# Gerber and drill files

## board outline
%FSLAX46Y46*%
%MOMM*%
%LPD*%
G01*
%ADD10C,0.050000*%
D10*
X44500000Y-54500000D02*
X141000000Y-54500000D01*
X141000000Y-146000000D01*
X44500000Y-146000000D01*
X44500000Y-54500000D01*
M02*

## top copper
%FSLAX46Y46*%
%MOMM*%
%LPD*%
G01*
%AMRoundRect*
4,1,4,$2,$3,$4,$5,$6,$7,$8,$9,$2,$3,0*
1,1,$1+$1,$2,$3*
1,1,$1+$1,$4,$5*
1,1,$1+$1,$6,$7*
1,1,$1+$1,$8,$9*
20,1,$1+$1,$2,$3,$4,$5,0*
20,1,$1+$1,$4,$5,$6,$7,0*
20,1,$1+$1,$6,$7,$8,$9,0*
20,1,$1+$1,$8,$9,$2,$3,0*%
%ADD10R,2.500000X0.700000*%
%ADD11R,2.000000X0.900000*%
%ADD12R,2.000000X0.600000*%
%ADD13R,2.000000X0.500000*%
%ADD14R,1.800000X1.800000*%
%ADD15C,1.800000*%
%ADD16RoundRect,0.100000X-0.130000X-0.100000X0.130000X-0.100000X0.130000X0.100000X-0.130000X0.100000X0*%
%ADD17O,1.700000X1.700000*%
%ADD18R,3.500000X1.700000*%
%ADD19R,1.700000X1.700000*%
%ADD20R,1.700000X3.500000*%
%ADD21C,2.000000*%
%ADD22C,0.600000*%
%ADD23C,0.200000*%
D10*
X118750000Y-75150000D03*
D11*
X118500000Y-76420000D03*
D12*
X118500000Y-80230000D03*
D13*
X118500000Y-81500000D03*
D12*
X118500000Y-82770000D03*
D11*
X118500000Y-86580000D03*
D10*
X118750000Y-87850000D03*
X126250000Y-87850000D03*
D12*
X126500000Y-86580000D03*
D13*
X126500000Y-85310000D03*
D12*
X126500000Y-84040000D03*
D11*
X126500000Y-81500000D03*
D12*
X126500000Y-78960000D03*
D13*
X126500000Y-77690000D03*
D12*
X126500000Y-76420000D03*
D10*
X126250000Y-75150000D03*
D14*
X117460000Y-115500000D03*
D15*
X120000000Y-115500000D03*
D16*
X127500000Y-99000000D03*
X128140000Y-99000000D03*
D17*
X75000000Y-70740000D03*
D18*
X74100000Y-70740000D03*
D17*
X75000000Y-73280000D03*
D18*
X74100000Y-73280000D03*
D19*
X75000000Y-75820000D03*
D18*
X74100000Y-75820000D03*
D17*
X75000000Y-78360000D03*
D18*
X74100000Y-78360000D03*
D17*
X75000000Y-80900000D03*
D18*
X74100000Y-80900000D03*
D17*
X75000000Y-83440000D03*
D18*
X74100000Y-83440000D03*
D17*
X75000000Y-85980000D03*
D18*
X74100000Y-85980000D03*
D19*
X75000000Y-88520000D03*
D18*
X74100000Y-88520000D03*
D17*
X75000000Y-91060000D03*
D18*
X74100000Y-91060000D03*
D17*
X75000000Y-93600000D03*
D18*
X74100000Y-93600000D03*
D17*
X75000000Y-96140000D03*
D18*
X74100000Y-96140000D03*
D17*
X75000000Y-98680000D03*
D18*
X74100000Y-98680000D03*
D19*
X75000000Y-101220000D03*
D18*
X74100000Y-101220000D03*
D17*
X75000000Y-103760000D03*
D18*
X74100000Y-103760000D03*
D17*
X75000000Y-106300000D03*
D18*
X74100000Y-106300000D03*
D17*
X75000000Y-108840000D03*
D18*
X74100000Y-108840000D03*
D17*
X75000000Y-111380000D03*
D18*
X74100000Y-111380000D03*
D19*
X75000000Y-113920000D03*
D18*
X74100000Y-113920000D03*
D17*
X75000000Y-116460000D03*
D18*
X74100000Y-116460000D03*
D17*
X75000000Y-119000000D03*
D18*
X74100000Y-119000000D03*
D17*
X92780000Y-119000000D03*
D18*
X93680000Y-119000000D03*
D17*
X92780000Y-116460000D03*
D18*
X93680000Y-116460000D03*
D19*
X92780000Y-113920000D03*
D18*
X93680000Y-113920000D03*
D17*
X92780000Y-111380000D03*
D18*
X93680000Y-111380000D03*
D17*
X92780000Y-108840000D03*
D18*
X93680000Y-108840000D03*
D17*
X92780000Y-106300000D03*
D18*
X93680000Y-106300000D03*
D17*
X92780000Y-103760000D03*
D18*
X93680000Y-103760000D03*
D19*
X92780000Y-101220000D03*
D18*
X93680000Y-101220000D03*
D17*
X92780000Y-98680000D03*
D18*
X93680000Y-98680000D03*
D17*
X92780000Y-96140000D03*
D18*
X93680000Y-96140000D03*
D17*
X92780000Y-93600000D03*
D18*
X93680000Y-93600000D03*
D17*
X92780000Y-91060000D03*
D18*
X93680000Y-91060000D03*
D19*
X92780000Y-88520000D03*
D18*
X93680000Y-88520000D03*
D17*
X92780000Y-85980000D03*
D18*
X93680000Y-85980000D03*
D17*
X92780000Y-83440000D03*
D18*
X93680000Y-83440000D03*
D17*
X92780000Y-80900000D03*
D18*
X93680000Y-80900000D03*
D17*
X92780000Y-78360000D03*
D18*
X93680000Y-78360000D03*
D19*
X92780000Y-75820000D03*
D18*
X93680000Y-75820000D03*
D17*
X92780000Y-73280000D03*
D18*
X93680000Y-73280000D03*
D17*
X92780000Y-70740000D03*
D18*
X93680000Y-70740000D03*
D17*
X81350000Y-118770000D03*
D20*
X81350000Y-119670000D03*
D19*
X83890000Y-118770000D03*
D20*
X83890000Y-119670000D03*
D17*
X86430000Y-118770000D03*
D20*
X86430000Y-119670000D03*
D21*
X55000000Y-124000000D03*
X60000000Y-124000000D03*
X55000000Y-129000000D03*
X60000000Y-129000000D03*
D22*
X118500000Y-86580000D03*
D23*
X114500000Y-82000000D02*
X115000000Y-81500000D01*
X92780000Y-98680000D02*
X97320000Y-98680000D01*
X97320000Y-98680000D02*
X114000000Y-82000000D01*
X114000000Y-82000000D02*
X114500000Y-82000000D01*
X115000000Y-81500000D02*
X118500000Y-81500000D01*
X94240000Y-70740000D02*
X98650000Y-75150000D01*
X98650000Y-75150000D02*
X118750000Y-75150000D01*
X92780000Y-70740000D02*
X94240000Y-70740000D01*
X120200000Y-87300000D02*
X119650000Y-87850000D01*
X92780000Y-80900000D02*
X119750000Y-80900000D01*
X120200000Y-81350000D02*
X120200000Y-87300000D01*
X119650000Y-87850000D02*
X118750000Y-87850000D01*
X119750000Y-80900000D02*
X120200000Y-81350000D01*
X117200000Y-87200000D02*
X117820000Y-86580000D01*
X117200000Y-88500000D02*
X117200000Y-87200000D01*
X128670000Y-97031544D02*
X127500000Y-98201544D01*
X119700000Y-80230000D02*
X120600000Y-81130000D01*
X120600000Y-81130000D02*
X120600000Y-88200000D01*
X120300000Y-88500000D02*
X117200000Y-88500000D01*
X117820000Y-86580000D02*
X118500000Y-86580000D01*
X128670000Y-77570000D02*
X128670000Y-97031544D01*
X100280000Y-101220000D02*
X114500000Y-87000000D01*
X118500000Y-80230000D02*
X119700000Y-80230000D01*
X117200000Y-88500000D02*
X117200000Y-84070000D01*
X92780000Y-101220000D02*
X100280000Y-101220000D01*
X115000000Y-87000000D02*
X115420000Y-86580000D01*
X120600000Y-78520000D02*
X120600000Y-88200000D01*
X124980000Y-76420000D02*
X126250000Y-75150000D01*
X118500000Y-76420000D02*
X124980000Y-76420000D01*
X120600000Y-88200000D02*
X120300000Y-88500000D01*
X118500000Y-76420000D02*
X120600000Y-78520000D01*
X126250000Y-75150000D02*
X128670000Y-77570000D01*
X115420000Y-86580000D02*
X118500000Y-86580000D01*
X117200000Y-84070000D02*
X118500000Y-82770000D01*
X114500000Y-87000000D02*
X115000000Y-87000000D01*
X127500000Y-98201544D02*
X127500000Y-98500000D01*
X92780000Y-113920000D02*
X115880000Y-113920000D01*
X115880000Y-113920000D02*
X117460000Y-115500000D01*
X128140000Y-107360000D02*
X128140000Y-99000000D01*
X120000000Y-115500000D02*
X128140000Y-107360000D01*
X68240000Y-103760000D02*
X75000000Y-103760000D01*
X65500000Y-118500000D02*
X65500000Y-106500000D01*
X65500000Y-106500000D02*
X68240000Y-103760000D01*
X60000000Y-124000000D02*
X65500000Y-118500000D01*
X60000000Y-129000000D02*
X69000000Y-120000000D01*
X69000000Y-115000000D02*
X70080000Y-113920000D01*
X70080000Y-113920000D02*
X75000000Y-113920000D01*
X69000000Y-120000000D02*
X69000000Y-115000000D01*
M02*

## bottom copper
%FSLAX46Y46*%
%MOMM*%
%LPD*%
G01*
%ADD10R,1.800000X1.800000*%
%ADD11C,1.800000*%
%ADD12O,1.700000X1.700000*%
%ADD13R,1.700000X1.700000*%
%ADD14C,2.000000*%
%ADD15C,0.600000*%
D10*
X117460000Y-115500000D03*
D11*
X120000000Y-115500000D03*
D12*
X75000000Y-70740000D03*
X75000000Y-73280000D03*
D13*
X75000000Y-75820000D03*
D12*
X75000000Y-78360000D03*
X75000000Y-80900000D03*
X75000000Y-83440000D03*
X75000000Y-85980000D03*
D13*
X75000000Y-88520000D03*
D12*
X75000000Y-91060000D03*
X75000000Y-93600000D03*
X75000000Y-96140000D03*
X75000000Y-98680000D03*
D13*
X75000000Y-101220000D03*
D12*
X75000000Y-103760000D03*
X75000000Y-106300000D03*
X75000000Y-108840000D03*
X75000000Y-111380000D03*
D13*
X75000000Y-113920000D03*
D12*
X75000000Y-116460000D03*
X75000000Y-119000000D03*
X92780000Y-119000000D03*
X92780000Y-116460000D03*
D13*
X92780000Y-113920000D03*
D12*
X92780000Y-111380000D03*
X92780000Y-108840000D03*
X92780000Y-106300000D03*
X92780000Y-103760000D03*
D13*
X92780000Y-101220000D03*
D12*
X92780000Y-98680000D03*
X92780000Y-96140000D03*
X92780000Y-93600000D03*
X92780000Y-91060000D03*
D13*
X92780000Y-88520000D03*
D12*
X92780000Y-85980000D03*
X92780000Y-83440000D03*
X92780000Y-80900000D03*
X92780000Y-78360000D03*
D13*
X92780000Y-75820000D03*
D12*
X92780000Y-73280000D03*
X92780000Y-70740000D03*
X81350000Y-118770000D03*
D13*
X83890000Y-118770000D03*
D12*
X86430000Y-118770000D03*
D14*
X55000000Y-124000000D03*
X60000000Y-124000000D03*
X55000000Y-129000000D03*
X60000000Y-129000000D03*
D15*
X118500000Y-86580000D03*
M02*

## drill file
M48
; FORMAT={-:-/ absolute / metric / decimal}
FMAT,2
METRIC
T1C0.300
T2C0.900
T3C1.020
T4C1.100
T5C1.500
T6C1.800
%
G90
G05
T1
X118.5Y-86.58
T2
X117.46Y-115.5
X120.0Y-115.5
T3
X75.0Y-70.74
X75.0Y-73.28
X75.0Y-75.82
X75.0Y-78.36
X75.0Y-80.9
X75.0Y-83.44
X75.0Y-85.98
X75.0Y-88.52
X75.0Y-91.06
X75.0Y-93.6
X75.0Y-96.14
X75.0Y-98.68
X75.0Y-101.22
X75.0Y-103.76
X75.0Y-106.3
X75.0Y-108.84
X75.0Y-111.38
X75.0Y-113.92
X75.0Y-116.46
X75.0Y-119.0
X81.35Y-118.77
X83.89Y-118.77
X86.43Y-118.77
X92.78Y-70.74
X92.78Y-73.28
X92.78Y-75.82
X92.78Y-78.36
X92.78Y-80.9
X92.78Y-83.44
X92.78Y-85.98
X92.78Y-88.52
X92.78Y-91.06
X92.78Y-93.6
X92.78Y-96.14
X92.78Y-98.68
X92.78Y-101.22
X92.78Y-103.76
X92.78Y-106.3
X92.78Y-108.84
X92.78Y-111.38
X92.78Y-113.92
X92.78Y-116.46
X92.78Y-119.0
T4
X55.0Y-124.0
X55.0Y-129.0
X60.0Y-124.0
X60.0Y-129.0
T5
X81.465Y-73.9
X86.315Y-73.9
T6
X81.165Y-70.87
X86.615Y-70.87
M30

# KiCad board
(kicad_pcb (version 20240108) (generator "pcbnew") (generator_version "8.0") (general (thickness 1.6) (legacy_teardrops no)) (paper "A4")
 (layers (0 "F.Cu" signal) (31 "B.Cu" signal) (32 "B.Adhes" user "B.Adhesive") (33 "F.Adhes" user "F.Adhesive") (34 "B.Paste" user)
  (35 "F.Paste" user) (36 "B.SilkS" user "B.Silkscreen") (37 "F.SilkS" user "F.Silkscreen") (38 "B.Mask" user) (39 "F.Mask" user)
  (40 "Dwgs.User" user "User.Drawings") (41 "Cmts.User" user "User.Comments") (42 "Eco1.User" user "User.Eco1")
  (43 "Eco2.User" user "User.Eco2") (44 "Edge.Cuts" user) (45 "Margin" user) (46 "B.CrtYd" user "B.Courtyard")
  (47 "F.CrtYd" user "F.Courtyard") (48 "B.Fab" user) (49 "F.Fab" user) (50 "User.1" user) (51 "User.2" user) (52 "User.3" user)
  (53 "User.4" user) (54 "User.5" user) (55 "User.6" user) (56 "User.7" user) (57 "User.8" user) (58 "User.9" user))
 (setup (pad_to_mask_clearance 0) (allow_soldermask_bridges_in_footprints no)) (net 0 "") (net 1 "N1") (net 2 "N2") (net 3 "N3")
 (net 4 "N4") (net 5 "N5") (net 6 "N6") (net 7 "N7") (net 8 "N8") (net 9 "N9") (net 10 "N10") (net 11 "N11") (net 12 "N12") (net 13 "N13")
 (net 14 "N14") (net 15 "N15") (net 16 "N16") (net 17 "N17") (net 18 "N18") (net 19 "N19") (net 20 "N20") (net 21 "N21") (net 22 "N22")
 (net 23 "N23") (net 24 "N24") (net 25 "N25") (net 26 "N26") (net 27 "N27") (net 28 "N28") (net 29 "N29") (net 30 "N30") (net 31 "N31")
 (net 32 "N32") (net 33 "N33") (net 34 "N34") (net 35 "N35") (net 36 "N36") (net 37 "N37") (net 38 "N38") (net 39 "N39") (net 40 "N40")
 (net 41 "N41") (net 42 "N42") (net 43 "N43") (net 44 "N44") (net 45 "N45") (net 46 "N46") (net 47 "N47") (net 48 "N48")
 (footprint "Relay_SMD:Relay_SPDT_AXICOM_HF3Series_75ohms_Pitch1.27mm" (layer "F.Cu") (at 122.5 81.5)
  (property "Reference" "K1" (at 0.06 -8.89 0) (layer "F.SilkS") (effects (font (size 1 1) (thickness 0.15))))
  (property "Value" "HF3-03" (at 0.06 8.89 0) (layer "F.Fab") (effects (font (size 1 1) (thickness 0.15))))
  (pad "1" smd rect (at -3.75 -6.35) (size 2.5 0.7) (layers "F.Cu" "F.Paste" "F.Mask") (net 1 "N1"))
  (pad "2" smd rect (at -4 -5.08) (size 2 0.9) (layers "F.Cu" "F.Paste" "F.Mask") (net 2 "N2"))
  (pad "5" smd rect (at -4 -1.27) (size 2 0.6) (layers "F.Cu" "F.Paste" "F.Mask") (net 2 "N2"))
  (pad "6" smd rect (at -4 0) (size 2 0.5) (layers "F.Cu" "F.Paste" "F.Mask") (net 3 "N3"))
  (pad "7" smd rect (at -4 1.27) (size 2 0.6) (layers "F.Cu" "F.Paste" "F.Mask") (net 2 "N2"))
  (pad "10" smd rect (at -4 5.08) (size 2 0.9) (layers "F.Cu" "F.Paste" "F.Mask") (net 2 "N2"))
  (pad "11" smd rect (at -3.75 6.35) (size 2.5 0.7) (layers "F.Cu" "F.Paste" "F.Mask") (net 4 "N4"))
  (pad "12" smd rect (at 3.75 6.35) (size 2.5 0.7) (layers "F.Cu" "F.Paste" "F.Mask") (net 2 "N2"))
  (pad "13" smd rect (at 4 5.08) (size 2 0.6) (layers "F.Cu" "F.Paste" "F.Mask") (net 2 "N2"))
  (pad "14" smd rect (at 4 3.81) (size 2 0.5) (layers "F.Cu" "F.Paste" "F.Mask") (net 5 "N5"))
  (pad "15" smd rect (at 4 2.54) (size 2 0.6) (layers "F.Cu" "F.Paste" "F.Mask") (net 2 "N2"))
  (pad "17" smd rect (at 4 0) (size 2 0.9) (layers "F.Cu" "F.Paste" "F.Mask") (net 2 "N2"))
  (pad "19" smd rect (at 4 -2.54) (size 2 0.6) (layers "F.Cu" "F.Paste" "F.Mask") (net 2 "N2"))
  (pad "20" smd rect (at 4 -3.81) (size 2 0.5) (layers "F.Cu" "F.Paste" "F.Mask") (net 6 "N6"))
  (pad "21" smd rect (at 4 -5.08) (size 2 0.6) (layers "F.Cu" "F.Paste" "F.Mask") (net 2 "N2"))
  (pad "22" smd rect (at 3.75 -6.35) (size 2.5 0.7) (layers "F.Cu" "F.Paste" "F.Mask") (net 2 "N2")))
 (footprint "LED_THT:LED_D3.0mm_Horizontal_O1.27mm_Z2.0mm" (layer "F.Cu") (at 117.46 115.5)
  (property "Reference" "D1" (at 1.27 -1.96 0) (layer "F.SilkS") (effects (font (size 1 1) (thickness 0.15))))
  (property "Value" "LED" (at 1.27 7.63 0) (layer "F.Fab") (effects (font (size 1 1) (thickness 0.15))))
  (pad "1" thru_hole rect (at 0 0) (size 1.8 1.8) (drill 0.9) (layers "*.Cu" "*.Mask") (remove_unused_layers no) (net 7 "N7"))
  (pad "2" thru_hole circle (at 2.54 0) (size 1.8 1.8) (drill 0.9) (layers "*.Cu" "*.Mask") (remove_unused_layers no) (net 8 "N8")))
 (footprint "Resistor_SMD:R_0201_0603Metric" (layer "F.Cu") (at 127.82 99)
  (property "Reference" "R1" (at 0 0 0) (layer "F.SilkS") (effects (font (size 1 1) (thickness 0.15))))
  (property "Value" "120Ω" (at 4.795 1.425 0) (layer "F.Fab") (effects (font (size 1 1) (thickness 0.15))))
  (pad "" smd roundrect (at -0.345 0) (size 0.318 0.36) (layers "F.Paste") (roundrect_rratio 0.25))
  (pad "" smd roundrect (at 0.345 0) (size 0.318 0.36) (layers "F.Paste") (roundrect_rratio 0.25))
  (pad "1" smd roundrect (at -0.32 0) (size 0.46 0.4) (layers "F.Cu" "F.Mask") (roundrect_rratio 0.25) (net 6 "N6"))
  (pad "2" smd roundrect (at 0.32 0) (size 0.46 0.4) (layers "F.Cu" "F.Mask") (roundrect_rratio 0.25) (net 8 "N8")))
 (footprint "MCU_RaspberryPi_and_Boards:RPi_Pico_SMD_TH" (layer "F.Cu") (at 83.89 94.87)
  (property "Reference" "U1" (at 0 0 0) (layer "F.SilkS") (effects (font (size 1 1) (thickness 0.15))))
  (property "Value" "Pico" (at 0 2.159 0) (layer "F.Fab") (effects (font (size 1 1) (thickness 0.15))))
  (pad "" np_thru_hole oval (at -2.725 -24) (size 1.8 1.8) (drill 1.8) (layers "*.Cu" "*.Mask"))
  (pad "" np_thru_hole oval (at -2.425 -20.97) (size 1.5 1.5) (drill 1.5) (layers "*.Cu" "*.Mask"))
  (pad "" np_thru_hole oval (at 2.425 -20.97) (size 1.5 1.5) (drill 1.5) (layers "*.Cu" "*.Mask"))
  (pad "" np_thru_hole oval (at 2.725 -24) (size 1.8 1.8) (drill 1.8) (layers "*.Cu" "*.Mask"))
  (pad "1" thru_hole oval (at -8.89 -24.13) (size 1.7 1.7) (drill 1.02) (layers "*.Cu" "*.Mask") (remove_unused_layers no) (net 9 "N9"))
  (pad "1" smd rect (at -8.89 -24.13) (size 3.5 1.7) (drill (offset -0.9 0)) (layers "F.Cu" "F.Mask") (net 9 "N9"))
  (pad "2" thru_hole oval (at -8.89 -21.59) (size 1.7 1.7) (drill 1.02) (layers "*.Cu" "*.Mask") (remove_unused_layers no) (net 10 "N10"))
  (pad "2" smd rect (at -8.89 -21.59) (size 3.5 1.7) (drill (offset -0.9 0)) (layers "F.Cu" "F.Mask") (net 10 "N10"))
  (pad "3" thru_hole rect (at -8.89 -19.05) (size 1.7 1.7) (drill 1.02) (layers "*.Cu" "*.Mask") (remove_unused_layers no) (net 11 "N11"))
  (pad "3" smd rect (at -8.89 -19.05) (size 3.5 1.7) (drill (offset -0.9 0)) (layers "F.Cu" "F.Mask") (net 11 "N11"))
  (pad "4" thru_hole oval (at -8.89 -16.51) (size 1.7 1.7) (drill 1.02) (layers "*.Cu" "*.Mask") (remove_unused_layers no) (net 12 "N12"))
  (pad "4" smd rect (at -8.89 -16.51) (size 3.5 1.7) (drill (offset -0.9 0)) (layers "F.Cu" "F.Mask") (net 12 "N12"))
  (pad "5" thru_hole oval (at -8.89 -13.97) (size 1.7 1.7) (drill 1.02) (layers "*.Cu" "*.Mask") (remove_unused_layers no) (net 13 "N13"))
  (pad "5" smd rect (at -8.89 -13.97) (size 3.5 1.7) (drill (offset -0.9 0)) (layers "F.Cu" "F.Mask") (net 13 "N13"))
  (pad "6" thru_hole oval (at -8.89 -11.43) (size 1.7 1.7) (drill 1.02) (layers "*.Cu" "*.Mask") (remove_unused_layers no) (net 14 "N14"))
  (pad "6" smd rect (at -8.89 -11.43) (size 3.5 1.7) (drill (offset -0.9 0)) (layers "F.Cu" "F.Mask") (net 14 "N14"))
  (pad "7" thru_hole oval (at -8.89 -8.89) (size 1.7 1.7) (drill 1.02) (layers "*.Cu" "*.Mask") (remove_unused_layers no) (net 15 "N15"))
  (pad "7" smd rect (at -8.89 -8.89) (size 3.5 1.7) (drill (offset -0.9 0)) (layers "F.Cu" "F.Mask") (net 15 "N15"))
  (pad "8" thru_hole rect (at -8.89 -6.35) (size 1.7 1.7) (drill 1.02) (layers "*.Cu" "*.Mask") (remove_unused_layers no) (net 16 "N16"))
  (pad "8" smd rect (at -8.89 -6.35) (size 3.5 1.7) (drill (offset -0.9 0)) (layers "F.Cu" "F.Mask") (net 16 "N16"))
  (pad "9" thru_hole oval (at -8.89 -3.81) (size 1.7 1.7) (drill 1.02) (layers "*.Cu" "*.Mask") (remove_unused_layers no) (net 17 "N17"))
  (pad "9" smd rect (at -8.89 -3.81) (size 3.5 1.7) (drill (offset -0.9 0)) (layers "F.Cu" "F.Mask") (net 17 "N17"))
  (pad "10" thru_hole oval (at -8.89 -1.27) (size 1.7 1.7) (drill 1.02) (layers "*.Cu" "*.Mask") (remove_unused_layers no) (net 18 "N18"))
  (pad "10" smd rect (at -8.89 -1.27) (size 3.5 1.7) (drill (offset -0.9 0)) (layers "F.Cu" "F.Mask") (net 18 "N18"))
  (pad "11" thru_hole oval (at -8.89 1.27) (size 1.7 1.7) (drill 1.02) (layers "*.Cu" "*.Mask") (remove_unused_layers no) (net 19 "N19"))
  (pad "11" smd rect (at -8.89 1.27) (size 3.5 1.7) (drill (offset -0.9 0)) (layers "F.Cu" "F.Mask") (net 19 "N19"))
  (pad "12" thru_hole oval (at -8.89 3.81) (size 1.7 1.7) (drill 1.02) (layers "*.Cu" "*.Mask") (remove_unused_layers no) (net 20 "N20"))
  (pad "12" smd rect (at -8.89 3.81) (size 3.5 1.7) (drill (offset -0.9 0)) (layers "F.Cu" "F.Mask") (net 20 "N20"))
  (pad "13" thru_hole rect (at -8.89 6.35) (size 1.7 1.7) (drill 1.02) (layers "*.Cu" "*.Mask") (remove_unused_layers no) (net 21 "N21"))
  (pad "13" smd rect (at -8.89 6.35) (size 3.5 1.7) (drill (offset -0.9 0)) (layers "F.Cu" "F.Mask") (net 21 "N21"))
  (pad "14" thru_hole oval (at -8.89 8.89) (size 1.7 1.7) (drill 1.02) (layers "*.Cu" "*.Mask") (remove_unused_layers no) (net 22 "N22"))
  (pad "14" smd rect (at -8.89 8.89) (size 3.5 1.7) (drill (offset -0.9 0)) (layers "F.Cu" "F.Mask") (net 22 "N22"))
  (pad "15" thru_hole oval (at -8.89 11.43) (size 1.7 1.7) (drill 1.02) (layers "*.Cu" "*.Mask") (remove_unused_layers no) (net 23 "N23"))
  (pad "15" smd rect (at -8.89 11.43) (size 3.5 1.7) (drill (offset -0.9 0)) (layers "F.Cu" "F.Mask") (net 23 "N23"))
  (pad "16" thru_hole oval (at -8.89 13.97) (size 1.7 1.7) (drill 1.02) (layers "*.Cu" "*.Mask") (remove_unused_layers no) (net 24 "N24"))
  (pad "16" smd rect (at -8.89 13.97) (size 3.5 1.7) (drill (offset -0.9 0)) (layers "F.Cu" "F.Mask") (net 24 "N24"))
  (pad "17" thru_hole oval (at -8.89 16.51) (size 1.7 1.7) (drill 1.02) (layers "*.Cu" "*.Mask") (remove_unused_layers no) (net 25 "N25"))
  (pad "17" smd rect (at -8.89 16.51) (size 3.5 1.7) (drill (offset -0.9 0)) (layers "F.Cu" "F.Mask") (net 25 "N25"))
  (pad "18" thru_hole rect (at -8.89 19.05) (size 1.7 1.7) (drill 1.02) (layers "*.Cu" "*.Mask") (remove_unused_layers no) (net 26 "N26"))
  (pad "18" smd rect (at -8.89 19.05) (size 3.5 1.7) (drill (offset -0.9 0)) (layers "F.Cu" "F.Mask") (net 26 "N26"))
  (pad "19" thru_hole oval (at -8.89 21.59) (size 1.7 1.7) (drill 1.02) (layers "*.Cu" "*.Mask") (remove_unused_layers no) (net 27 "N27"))
  (pad "19" smd rect (at -8.89 21.59) (size 3.5 1.7) (drill (offset -0.9 0)) (layers "F.Cu" "F.Mask") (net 27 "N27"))
  (pad "20" thru_hole oval (at -8.89 24.13) (size 1.7 1.7) (drill 1.02) (layers "*.Cu" "*.Mask") (remove_unused_layers no) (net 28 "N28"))
  (pad "20" smd rect (at -8.89 24.13) (size 3.5 1.7) (drill (offset -0.9 0)) (layers "F.Cu" "F.Mask") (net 28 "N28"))
  (pad "21" thru_hole oval (at 8.89 24.13) (size 1.7 1.7) (drill 1.02) (layers "*.Cu" "*.Mask") (remove_unused_layers no) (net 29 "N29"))
  (pad "21" smd rect (at 8.89 24.13) (size 3.5 1.7) (drill (offset 0.9 0)) (layers "F.Cu" "F.Mask") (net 29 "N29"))
  (pad "22" thru_hole oval (at 8.89 21.59) (size 1.7 1.7) (drill 1.02) (layers "*.Cu" "*.Mask") (remove_unused_layers no) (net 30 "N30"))
  (pad "22" smd rect (at 8.89 21.59) (size 3.5 1.7) (drill (offset 0.9 0)) (layers "F.Cu" "F.Mask") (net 30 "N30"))
  (pad "23" thru_hole rect (at 8.89 19.05) (size 1.7 1.7) (drill 1.02) (layers "*.Cu" "*.Mask") (remove_unused_layers no) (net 7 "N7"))
  (pad "23" smd rect (at 8.89 19.05) (size 3.5 1.7) (drill (offset 0.9 0)) (layers "F.Cu" "F.Mask") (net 7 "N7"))
  (pad "24" thru_hole oval (at 8.89 16.51) (size 1.7 1.7) (drill 1.02) (layers "*.Cu" "*.Mask") (remove_unused_layers no) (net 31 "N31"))
  (pad "24" smd rect (at 8.89 16.51) (size 3.5 1.7) (drill (offset 0.9 0)) (layers "F.Cu" "F.Mask") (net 31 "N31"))
  (pad "25" thru_hole oval (at 8.89 13.97) (size 1.7 1.7) (drill 1.02) (layers "*.Cu" "*.Mask") (remove_unused_layers no) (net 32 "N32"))
  (pad "25" smd rect (at 8.89 13.97) (size 3.5 1.7) (drill (offset 0.9 0)) (layers "F.Cu" "F.Mask") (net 32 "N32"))
  (pad "26" thru_hole oval (at 8.89 11.43) (size 1.7 1.7) (drill 1.02) (layers "*.Cu" "*.Mask") (remove_unused_layers no) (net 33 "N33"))
  (pad "26" smd rect (at 8.89 11.43) (size 3.5 1.7) (drill (offset 0.9 0)) (layers "F.Cu" "F.Mask") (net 33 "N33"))
  (pad "27" thru_hole oval (at 8.89 8.89) (size 1.7 1.7) (drill 1.02) (layers "*.Cu" "*.Mask") (remove_unused_layers no) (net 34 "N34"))
  (pad "27" smd rect (at 8.89 8.89) (size 3.5 1.7) (drill (offset 0.9 0)) (layers "F.Cu" "F.Mask") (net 34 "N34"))
  (pad "28" thru_hole rect (at 8.89 6.35) (size 1.7 1.7) (drill 1.02) (layers "*.Cu" "*.Mask") (remove_unused_layers no) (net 2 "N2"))
  (pad "28" smd rect (at 8.89 6.35) (size 3.5 1.7) (drill (offset 0.9 0)) (layers "F.Cu" "F.Mask") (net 2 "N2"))
  (pad "29" thru_hole oval (at 8.89 3.81) (size 1.7 1.7) (drill 1.02) (layers "*.Cu" "*.Mask") (remove_unused_layers no) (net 3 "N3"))
  (pad "29" smd rect (at 8.89 3.81) (size 3.5 1.7) (drill (offset 0.9 0)) (layers "F.Cu" "F.Mask") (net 3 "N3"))
  (pad "30" thru_hole oval (at 8.89 1.27) (size 1.7 1.7) (drill 1.02) (layers "*.Cu" "*.Mask") (remove_unused_layers no) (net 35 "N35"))
  (pad "30" smd rect (at 8.89 1.27) (size 3.5 1.7) (drill (offset 0.9 0)) (layers "F.Cu" "F.Mask") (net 35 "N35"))
  (pad "31" thru_hole oval (at 8.89 -1.27) (size 1.7 1.7) (drill 1.02) (layers "*.Cu" "*.Mask") (remove_unused_layers no) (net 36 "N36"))
  (pad "31" smd rect (at 8.89 -1.27) (size 3.5 1.7) (drill (offset 0.9 0)) (layers "F.Cu" "F.Mask") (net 36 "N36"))
  (pad "32" thru_hole oval (at 8.89 -3.81) (size 1.7 1.7) (drill 1.02) (layers "*.Cu" "*.Mask") (remove_unused_layers no) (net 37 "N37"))
  (pad "32" smd rect (at 8.89 -3.81) (size 3.5 1.7) (drill (offset 0.9 0)) (layers "F.Cu" "F.Mask") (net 37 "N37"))
  (pad "33" thru_hole rect (at 8.89 -6.35) (size 1.7 1.7) (drill 1.02) (layers "*.Cu" "*.Mask") (remove_unused_layers no) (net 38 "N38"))
  (pad "33" smd rect (at 8.89 -6.35) (size 3.5 1.7) (drill (offset 0.9 0)) (layers "F.Cu" "F.Mask") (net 38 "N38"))
  (pad "34" thru_hole oval (at 8.89 -8.89) (size 1.7 1.7) (drill 1.02) (layers "*.Cu" "*.Mask") (remove_unused_layers no) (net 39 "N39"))
  (pad "34" smd rect (at 8.89 -8.89) (size 3.5 1.7) (drill (offset 0.9 0)) (layers "F.Cu" "F.Mask") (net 39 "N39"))
  (pad "35" thru_hole oval (at 8.89 -11.43) (size 1.7 1.7) (drill 1.02) (layers "*.Cu" "*.Mask") (remove_unused_layers no) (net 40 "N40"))
  (pad "35" smd rect (at 8.89 -11.43) (size 3.5 1.7) (drill (offset 0.9 0)) (layers "F.Cu" "F.Mask") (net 40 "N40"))
  (pad "36" thru_hole oval (at 8.89 -13.97) (size 1.7 1.7) (drill 1.02) (layers "*.Cu" "*.Mask") (remove_unused_layers no) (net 4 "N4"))
  (pad "36" smd rect (at 8.89 -13.97) (size 3.5 1.7) (drill (offset 0.9 0)) (layers "F.Cu" "F.Mask") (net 4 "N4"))
  (pad "37" thru_hole oval (at 8.89 -16.51) (size 1.7 1.7) (drill 1.02) (layers "*.Cu" "*.Mask") (remove_unused_layers no) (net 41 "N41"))
  (pad "37" smd rect (at 8.89 -16.51) (size 3.5 1.7) (drill (offset 0.9 0)) (layers "F.Cu" "F.Mask") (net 41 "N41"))
  (pad "38" thru_hole rect (at 8.89 -19.05) (size 1.7 1.7) (drill 1.02) (layers "*.Cu" "*.Mask") (remove_unused_layers no) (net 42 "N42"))
  (pad "38" smd rect (at 8.89 -19.05) (size 3.5 1.7) (drill (offset 0.9 0)) (layers "F.Cu" "F.Mask") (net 42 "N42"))
  (pad "39" thru_hole oval (at 8.89 -21.59) (size 1.7 1.7) (drill 1.02) (layers "*.Cu" "*.Mask") (remove_unused_layers no) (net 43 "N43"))
  (pad "39" smd rect (at 8.89 -21.59) (size 3.5 1.7) (drill (offset 0.9 0)) (layers "F.Cu" "F.Mask") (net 43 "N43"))
  (pad "40" thru_hole oval (at 8.89 -24.13) (size 1.7 1.7) (drill 1.02) (layers "*.Cu" "*.Mask") (remove_unused_layers no) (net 1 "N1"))
  (pad "40" smd rect (at 8.89 -24.13) (size 3.5 1.7) (drill (offset 0.9 0)) (layers "F.Cu" "F.Mask") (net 1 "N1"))
  (pad "41" thru_hole oval (at -2.54 23.9) (size 1.7 1.7) (drill 1.02) (layers "*.Cu" "*.Mask") (remove_unused_layers no) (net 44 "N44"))
  (pad "41" smd rect (at -2.54 23.9 90) (size 3.5 1.7) (drill (offset -0.9 0)) (layers "F.Cu" "F.Mask") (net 44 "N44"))
  (pad "42" thru_hole rect (at 0 23.9) (size 1.7 1.7) (drill 1.02) (layers "*.Cu" "*.Mask") (remove_unused_layers no) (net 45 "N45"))
  (pad "42" smd rect (at 0 23.9 90) (size 3.5 1.7) (drill (offset -0.9 0)) (layers "F.Cu" "F.Mask") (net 45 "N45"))
  (pad "43" thru_hole oval (at 2.54 23.9) (size 1.7 1.7) (drill 1.02) (layers "*.Cu" "*.Mask") (remove_unused_layers no) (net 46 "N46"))
  (pad "43" smd rect (at 2.54 23.9 90) (size 3.5 1.7) (drill (offset -0.9 0)) (layers "F.Cu" "F.Mask") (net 46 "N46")))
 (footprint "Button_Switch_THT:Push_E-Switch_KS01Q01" (layer "F.Cu") (at 55 124)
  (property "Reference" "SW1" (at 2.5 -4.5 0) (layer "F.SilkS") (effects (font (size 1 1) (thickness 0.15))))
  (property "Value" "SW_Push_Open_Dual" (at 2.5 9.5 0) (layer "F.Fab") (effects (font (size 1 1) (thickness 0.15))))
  (pad "1" thru_hole circle (at 0 0) (size 2 2) (drill 1.1) (layers "*.Cu" "*.Mask") (remove_unused_layers no) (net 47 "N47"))
  (pad "2" thru_hole circle (at 5 0) (size 2 2) (drill 1.1) (layers "*.Cu" "*.Mask") (remove_unused_layers no) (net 22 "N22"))
  (pad "3" thru_hole circle (at 0 5) (size 2 2) (drill 1.1) (layers "*.Cu" "*.Mask") (remove_unused_layers no) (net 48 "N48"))
  (pad "4" thru_hole circle (at 5 5) (size 2 2) (drill 1.1) (layers "*.Cu" "*.Mask") (remove_unused_layers no) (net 26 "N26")))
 (gr_rect (start 44.5 54.5) (end 141 146) (stroke (width 0.05) (type default)) (fill none) (layer "Edge.Cuts"))
 (segment (start 114.5 82) (end 115 81.5) (width 0.2) (layer "F.Cu") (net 3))
 (segment (start 92.78 98.68) (end 97.32 98.68) (width 0.2) (layer "F.Cu") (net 3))
 (segment (start 97.32 98.68) (end 114 82) (width 0.2) (layer "F.Cu") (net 3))
 (segment (start 114 82) (end 114.5 82) (width 0.2) (layer "F.Cu") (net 3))
 (segment (start 115 81.5) (end 118.5 81.5) (width 0.2) (layer "F.Cu") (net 3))
 (segment (start 94.24 70.74) (end 98.65 75.15) (width 0.2) (layer "F.Cu") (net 1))
 (segment (start 98.65 75.15) (end 118.75 75.15) (width 0.2) (layer "F.Cu") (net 1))
 (segment (start 92.78 70.74) (end 94.24 70.74) (width 0.2) (layer "F.Cu") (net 1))
 (segment (start 120.2 87.3) (end 119.65 87.85) (width 0.2) (layer "F.Cu") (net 4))
 (segment (start 92.78 80.9) (end 119.75 80.9) (width 0.2) (layer "F.Cu") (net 4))
 (segment (start 120.2 81.35) (end 120.2 87.3) (width 0.2) (layer "F.Cu") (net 4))
 (segment (start 119.65 87.85) (end 118.75 87.85) (width 0.2) (layer "F.Cu") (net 4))
 (segment (start 119.75 80.9) (end 120.2 81.35) (width 0.2) (layer "F.Cu") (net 4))
 (segment (start 117.2 87.2) (end 117.82 86.58) (width 0.2) (layer "F.Cu") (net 2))
 (segment (start 117.2 88.5) (end 117.2 87.2) (width 0.2) (layer "F.Cu") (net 2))
 (segment (start 128.67 97.031544) (end 127.5 98.201544) (width 0.2) (layer "F.Cu") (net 2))
 (segment (start 119.7 80.23) (end 120.6 81.13) (width 0.2) (layer "F.Cu") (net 2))
 (segment (start 120.6 81.13) (end 120.6 88.2) (width 0.2) (layer "F.Cu") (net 2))
 (segment (start 120.3 88.5) (end 117.2 88.5) (width 0.2) (layer "F.Cu") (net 2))
 (segment (start 117.82 86.58) (end 118.5 86.58) (width 0.2) (layer "F.Cu") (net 2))
 (segment (start 128.67 77.57) (end 128.67 97.031544) (width 0.2) (layer "F.Cu") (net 2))
 (segment (start 100.28 101.22) (end 114.5 87) (width 0.2) (layer "F.Cu") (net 2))
 (segment (start 118.5 80.23) (end 119.7 80.23) (width 0.2) (layer "F.Cu") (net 2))
 (segment (start 117.2 88.5) (end 117.2 84.07) (width 0.2) (layer "F.Cu") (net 2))
 (segment (start 92.78 101.22) (end 100.28 101.22) (width 0.2) (layer "F.Cu") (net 2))
 (segment (start 115 87) (end 115.42 86.58) (width 0.2) (layer "F.Cu") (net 2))
 (segment (start 120.6 78.52) (end 120.6 88.2) (width 0.2) (layer "F.Cu") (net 2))
 (segment (start 124.98 76.42) (end 126.25 75.15) (width 0.2) (layer "F.Cu") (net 2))
 (segment (start 118.5 76.42) (end 124.98 76.42) (width 0.2) (layer "F.Cu") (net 2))
 (segment (start 120.6 88.2) (end 120.3 88.5) (width 0.2) (layer "F.Cu") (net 2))
 (segment (start 118.5 76.42) (end 120.6 78.52) (width 0.2) (layer "F.Cu") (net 2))
 (segment (start 126.25 75.15) (end 128.67 77.57) (width 0.2) (layer "F.Cu") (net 2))
 (segment (start 115.42 86.58) (end 118.5 86.58) (width 0.2) (layer "F.Cu") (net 2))
 (segment (start 117.2 84.07) (end 118.5 82.77) (width 0.2) (layer "F.Cu") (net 2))
 (segment (start 114.5 87) (end 115 87) (width 0.2) (layer "F.Cu") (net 2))
 (segment (start 127.5 98.201544) (end 127.5 98.5) (width 0.2) (layer "F.Cu") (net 2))
 (via (at 118.5 86.58) (size 0.6) (drill 0.3) (layers "F.Cu" "B.Cu") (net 2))
 (segment (start 92.78 113.92) (end 115.88 113.92) (width 0.2) (layer "F.Cu") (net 7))
 (segment (start 115.88 113.92) (end 117.46 115.5) (width 0.2) (layer "F.Cu") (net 7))
 (segment (start 128.14 107.36) (end 128.14 99) (width 0.2) (layer "F.Cu") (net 8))
 (segment (start 120 115.5) (end 128.14 107.36) (width 0.2) (layer "F.Cu") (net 8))
 (segment (start 68.24 103.76) (end 75 103.76) (width 0.2) (layer "F.Cu") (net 22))
 (segment (start 65.5 118.5) (end 65.5 106.5) (width 0.2) (layer "F.Cu") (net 22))
 (segment (start 65.5 106.5) (end 68.24 103.76) (width 0.2) (layer "F.Cu") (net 22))
 (segment (start 60 124) (end 65.5 118.5) (width 0.2) (layer "F.Cu") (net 22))
 (segment (start 60 129) (end 69 120) (width 0.2) (layer "F.Cu") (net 26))
 (segment (start 69 115) (end 70.08 113.92) (width 0.2) (layer "F.Cu") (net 26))
 (segment (start 70.08 113.92) (end 75 113.92) (width 0.2) (layer "F.Cu") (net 26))
 (segment (start 69 120) (end 69 115) (width 0.2) (layer "F.Cu") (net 26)))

